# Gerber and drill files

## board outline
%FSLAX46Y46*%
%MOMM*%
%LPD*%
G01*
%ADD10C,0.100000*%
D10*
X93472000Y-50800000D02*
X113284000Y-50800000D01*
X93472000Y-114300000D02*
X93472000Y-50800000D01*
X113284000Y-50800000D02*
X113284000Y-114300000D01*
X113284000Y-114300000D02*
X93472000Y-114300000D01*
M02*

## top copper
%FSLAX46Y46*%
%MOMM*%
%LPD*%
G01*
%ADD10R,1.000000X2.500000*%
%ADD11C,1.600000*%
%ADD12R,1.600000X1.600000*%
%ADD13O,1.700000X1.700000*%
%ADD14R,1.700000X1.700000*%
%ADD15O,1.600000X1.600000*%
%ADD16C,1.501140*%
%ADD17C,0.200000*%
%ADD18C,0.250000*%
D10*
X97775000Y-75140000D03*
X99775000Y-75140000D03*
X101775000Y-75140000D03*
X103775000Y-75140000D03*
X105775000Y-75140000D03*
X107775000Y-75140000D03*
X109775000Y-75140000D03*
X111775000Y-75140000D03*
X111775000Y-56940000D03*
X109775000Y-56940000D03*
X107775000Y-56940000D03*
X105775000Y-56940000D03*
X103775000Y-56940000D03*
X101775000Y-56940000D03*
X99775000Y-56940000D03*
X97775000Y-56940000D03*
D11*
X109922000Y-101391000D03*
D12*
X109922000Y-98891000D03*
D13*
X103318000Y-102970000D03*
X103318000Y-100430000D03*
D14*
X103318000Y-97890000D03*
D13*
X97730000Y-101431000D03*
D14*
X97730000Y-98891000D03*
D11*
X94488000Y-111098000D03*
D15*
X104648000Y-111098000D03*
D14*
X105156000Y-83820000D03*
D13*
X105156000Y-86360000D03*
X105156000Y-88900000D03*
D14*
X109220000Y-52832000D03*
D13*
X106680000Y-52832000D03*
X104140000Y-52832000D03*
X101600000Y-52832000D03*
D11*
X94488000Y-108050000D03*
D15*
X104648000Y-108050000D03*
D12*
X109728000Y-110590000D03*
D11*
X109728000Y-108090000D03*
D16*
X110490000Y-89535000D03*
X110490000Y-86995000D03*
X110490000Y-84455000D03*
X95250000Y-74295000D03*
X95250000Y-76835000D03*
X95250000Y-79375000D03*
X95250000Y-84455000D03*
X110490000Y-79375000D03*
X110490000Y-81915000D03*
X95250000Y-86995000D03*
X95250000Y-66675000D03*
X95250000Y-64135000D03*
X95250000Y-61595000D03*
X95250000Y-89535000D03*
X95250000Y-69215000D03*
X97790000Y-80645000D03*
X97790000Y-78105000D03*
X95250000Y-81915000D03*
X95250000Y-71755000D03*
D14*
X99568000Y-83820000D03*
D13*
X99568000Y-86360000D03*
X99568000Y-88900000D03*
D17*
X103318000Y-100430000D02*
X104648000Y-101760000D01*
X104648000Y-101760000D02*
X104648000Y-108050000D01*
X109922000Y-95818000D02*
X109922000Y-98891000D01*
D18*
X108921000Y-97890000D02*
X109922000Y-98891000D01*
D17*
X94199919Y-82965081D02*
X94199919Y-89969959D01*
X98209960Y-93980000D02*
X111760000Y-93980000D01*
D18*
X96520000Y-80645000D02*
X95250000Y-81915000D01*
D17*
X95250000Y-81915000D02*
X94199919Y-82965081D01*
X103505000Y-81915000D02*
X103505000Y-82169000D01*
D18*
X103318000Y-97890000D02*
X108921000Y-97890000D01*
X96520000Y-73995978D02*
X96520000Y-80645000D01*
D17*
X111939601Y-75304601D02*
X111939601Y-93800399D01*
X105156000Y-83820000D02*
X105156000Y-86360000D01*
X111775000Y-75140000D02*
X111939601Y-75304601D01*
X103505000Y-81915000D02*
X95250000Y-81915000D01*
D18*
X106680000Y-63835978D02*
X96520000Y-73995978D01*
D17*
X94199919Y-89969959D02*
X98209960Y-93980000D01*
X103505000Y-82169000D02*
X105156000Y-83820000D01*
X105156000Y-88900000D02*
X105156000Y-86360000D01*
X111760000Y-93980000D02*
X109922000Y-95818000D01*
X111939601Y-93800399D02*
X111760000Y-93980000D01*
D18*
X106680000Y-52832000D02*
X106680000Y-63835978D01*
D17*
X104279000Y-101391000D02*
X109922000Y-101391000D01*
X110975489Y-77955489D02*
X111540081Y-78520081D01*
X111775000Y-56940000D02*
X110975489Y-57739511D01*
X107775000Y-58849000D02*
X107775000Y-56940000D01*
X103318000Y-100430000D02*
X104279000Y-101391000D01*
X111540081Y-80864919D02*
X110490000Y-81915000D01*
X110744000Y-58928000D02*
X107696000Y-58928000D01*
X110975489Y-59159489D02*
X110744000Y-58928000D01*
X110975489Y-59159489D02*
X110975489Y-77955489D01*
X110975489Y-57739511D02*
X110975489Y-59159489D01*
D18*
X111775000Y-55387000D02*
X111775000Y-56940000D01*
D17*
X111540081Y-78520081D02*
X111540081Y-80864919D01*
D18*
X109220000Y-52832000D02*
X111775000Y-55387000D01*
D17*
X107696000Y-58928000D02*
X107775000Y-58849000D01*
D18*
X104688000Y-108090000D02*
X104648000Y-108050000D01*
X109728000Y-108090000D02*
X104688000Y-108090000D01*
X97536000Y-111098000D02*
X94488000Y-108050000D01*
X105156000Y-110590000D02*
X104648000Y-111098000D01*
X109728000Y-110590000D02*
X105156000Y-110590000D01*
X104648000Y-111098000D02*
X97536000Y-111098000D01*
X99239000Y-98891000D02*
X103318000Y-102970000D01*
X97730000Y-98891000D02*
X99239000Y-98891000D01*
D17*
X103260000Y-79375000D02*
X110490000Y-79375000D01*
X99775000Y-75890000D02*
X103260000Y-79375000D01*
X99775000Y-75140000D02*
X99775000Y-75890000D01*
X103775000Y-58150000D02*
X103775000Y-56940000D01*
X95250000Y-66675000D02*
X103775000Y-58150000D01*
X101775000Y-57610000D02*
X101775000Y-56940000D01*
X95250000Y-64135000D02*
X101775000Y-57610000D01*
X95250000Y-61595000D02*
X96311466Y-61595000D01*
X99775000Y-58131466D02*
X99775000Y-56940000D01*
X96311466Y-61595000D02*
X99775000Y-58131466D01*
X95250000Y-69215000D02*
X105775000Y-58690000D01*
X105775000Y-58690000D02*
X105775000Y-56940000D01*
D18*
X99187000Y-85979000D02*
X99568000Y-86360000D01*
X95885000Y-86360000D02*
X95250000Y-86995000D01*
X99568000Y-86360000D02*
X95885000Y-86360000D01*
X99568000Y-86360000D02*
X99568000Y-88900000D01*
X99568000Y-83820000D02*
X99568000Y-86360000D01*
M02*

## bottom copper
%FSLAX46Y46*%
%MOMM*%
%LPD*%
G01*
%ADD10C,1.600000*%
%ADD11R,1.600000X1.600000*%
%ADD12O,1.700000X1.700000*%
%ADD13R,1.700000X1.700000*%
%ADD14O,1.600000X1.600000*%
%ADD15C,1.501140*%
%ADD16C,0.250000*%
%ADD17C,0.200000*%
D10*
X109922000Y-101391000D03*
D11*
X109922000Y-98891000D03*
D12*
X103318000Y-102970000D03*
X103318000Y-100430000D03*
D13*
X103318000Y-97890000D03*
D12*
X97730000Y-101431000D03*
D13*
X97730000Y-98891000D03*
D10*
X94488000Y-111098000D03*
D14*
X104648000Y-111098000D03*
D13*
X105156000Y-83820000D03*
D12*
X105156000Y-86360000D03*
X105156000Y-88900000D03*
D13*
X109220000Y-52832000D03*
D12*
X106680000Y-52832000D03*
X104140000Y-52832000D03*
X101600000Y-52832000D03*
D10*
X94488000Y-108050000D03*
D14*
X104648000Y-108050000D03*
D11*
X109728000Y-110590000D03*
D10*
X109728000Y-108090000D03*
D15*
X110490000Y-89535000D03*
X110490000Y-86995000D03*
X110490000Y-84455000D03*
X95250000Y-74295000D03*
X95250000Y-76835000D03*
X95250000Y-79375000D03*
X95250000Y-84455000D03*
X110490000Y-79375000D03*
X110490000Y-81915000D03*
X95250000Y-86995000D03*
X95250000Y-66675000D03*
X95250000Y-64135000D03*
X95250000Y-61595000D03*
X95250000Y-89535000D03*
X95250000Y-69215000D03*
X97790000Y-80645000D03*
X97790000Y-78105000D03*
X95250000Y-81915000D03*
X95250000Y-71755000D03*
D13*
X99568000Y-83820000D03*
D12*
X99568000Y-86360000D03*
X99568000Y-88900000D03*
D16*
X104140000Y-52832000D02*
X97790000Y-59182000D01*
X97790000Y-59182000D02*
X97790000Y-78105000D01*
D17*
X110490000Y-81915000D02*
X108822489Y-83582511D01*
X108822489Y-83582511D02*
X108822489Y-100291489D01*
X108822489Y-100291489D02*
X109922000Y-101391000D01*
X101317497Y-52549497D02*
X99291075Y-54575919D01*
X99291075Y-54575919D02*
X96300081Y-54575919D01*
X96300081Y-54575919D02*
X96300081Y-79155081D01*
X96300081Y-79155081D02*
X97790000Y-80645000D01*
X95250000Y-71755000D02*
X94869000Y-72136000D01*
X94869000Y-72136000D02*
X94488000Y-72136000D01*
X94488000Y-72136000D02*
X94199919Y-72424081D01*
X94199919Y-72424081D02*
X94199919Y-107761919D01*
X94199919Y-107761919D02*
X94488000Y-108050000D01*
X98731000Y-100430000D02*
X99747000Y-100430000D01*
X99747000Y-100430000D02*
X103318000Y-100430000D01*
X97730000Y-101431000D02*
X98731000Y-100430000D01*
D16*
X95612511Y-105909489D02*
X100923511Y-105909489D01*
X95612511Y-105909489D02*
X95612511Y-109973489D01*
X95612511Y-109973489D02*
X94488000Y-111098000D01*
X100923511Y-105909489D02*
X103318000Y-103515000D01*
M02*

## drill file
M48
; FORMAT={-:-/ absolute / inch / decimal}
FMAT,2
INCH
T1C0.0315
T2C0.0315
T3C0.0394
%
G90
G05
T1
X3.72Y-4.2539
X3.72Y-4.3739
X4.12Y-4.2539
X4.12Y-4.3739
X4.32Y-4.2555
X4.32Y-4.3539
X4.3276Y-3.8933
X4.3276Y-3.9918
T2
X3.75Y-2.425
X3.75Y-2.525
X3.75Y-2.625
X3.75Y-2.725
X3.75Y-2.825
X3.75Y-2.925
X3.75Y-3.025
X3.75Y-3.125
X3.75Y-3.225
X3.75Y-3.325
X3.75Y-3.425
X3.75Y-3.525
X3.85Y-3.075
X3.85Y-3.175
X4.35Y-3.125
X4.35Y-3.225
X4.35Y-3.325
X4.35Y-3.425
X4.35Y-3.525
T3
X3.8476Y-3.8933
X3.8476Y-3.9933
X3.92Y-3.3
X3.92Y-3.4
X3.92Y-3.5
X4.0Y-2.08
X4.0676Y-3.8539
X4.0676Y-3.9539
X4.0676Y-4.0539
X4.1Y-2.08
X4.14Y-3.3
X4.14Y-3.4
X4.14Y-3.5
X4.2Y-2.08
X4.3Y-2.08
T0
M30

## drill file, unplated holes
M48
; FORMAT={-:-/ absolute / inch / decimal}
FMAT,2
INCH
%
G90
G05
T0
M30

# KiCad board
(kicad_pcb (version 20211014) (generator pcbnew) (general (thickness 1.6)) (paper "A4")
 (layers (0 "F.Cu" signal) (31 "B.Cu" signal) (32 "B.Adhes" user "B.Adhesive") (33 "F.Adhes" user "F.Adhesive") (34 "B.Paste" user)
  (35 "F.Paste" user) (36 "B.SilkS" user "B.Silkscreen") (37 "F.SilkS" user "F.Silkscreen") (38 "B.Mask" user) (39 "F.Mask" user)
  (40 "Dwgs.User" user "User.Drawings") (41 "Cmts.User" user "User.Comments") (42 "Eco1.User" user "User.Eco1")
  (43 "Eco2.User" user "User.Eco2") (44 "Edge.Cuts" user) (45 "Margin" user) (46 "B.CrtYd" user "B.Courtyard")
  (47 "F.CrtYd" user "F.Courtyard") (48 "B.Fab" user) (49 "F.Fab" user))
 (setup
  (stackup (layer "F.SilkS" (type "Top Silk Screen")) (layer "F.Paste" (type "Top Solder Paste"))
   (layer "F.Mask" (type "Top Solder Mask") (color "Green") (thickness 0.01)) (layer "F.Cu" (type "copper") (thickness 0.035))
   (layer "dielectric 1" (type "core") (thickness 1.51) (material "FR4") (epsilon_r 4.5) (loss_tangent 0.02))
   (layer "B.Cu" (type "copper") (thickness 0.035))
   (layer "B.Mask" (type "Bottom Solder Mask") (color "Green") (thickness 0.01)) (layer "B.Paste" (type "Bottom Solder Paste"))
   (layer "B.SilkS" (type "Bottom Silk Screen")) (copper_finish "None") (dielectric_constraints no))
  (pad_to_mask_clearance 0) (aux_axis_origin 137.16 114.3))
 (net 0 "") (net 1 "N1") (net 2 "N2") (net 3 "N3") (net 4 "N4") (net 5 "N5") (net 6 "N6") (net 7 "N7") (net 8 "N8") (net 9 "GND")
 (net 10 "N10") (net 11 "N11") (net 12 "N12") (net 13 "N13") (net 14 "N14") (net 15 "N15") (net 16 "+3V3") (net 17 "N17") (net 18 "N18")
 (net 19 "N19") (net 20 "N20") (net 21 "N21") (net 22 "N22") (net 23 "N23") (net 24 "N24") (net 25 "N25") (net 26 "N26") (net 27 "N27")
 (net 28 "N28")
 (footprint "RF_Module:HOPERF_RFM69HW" (layer "F.Cu") (at 104.775 66.04 90)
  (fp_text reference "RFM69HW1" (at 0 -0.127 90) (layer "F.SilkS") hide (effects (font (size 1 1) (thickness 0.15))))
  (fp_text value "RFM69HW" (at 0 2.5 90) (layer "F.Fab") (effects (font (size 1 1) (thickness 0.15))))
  (pad "1" smd rect (at -9.1 -7 90) (size 2.5 1) (layers "F.Cu" "F.Paste" "F.Mask") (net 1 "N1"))
  (pad "2" smd rect (at -9.1 -5 90) (size 2.5 1) (layers "F.Cu" "F.Paste" "F.Mask") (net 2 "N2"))
  (pad "3" smd rect (at -9.1 -3 90) (size 2.5 1) (layers "F.Cu" "F.Paste" "F.Mask") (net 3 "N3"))
  (pad "4" smd rect (at -9.1 -1 90) (size 2.5 1) (layers "F.Cu" "F.Paste" "F.Mask") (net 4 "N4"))
  (pad "5" smd rect (at -9.1 1 90) (size 2.5 1) (layers "F.Cu" "F.Paste" "F.Mask") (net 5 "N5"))
  (pad "6" smd rect (at -9.1 3 90) (size 2.5 1) (layers "F.Cu" "F.Paste" "F.Mask") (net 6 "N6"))
  (pad "7" smd rect (at -9.1 5 90) (size 2.5 1) (layers "F.Cu" "F.Paste" "F.Mask") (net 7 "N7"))
  (pad "8" smd rect (at -9.1 7 90) (size 2.5 1) (layers "F.Cu" "F.Paste" "F.Mask") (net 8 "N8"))
  (pad "9" smd rect (at 9.1 7 90) (size 2.5 1) (layers "F.Cu" "F.Paste" "F.Mask") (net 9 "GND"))
  (pad "10" smd rect (at 9.1 5 90) (size 2.5 1) (layers "F.Cu" "F.Paste" "F.Mask") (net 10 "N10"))
  (pad "11" smd rect (at 9.1 3 90) (size 2.5 1) (layers "F.Cu" "F.Paste" "F.Mask") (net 9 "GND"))
  (pad "12" smd rect (at 9.1 1 90) (size 2.5 1) (layers "F.Cu" "F.Paste" "F.Mask") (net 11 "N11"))
  (pad "13" smd rect (at 9.1 -1 90) (size 2.5 1) (layers "F.Cu" "F.Paste" "F.Mask") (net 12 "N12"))
  (pad "14" smd rect (at 9.1 -3 90) (size 2.5 1) (layers "F.Cu" "F.Paste" "F.Mask") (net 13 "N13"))
  (pad "15" smd rect (at 9.1 -5 90) (size 2.5 1) (layers "F.Cu" "F.Paste" "F.Mask") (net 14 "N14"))
  (pad "16" smd rect (at 9.1 -7 90) (size 2.5 1) (layers "F.Cu" "F.Paste" "F.Mask") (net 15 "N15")))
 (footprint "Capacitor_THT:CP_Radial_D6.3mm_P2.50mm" (layer "F.Cu") (at 109.922 98.891 -90)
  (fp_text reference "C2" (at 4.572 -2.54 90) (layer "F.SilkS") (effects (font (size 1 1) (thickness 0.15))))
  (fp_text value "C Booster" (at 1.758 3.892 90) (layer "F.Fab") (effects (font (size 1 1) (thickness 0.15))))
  (pad "1" thru_hole rect (at 0 0 270) (size 1.6 1.6) (drill 0.8) (layers *.Cu *.Mask) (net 8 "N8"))
  (pad "2" thru_hole circle (at 2.5 0 270) (size 1.6 1.6) (drill 0.8) (layers *.Cu *.Mask) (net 9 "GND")))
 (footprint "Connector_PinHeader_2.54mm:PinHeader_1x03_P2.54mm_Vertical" (layer "F.Cu") (at 103.318 97.89)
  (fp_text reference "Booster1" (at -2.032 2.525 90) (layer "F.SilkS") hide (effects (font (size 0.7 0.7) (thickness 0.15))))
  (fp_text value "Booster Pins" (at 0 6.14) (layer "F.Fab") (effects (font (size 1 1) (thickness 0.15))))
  (pad "1" thru_hole rect (at 0 0) (size 1.7 1.7) (drill 1) (layers *.Cu *.Mask) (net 8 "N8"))
  (pad "2" thru_hole oval (at 0 2.54) (size 1.7 1.7) (drill 1) (layers *.Cu *.Mask) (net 9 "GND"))
  (pad "3" thru_hole oval (at 0 5.08) (size 1.7 1.7) (drill 1) (layers *.Cu *.Mask) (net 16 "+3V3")))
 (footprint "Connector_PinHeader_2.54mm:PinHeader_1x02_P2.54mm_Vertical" (layer "F.Cu") (at 97.73 98.891)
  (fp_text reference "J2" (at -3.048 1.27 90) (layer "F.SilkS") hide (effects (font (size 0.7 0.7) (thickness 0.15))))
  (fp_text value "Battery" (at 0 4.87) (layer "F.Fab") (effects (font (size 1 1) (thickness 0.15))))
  (pad "1" thru_hole rect (at 0 0) (size 1.7 1.7) (drill 1) (layers *.Cu *.Mask) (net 16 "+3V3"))
  (pad "2" thru_hole oval (at 0 2.54) (size 1.7 1.7) (drill 1) (layers *.Cu *.Mask) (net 9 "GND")))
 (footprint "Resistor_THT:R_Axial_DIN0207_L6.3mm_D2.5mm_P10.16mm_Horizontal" (layer "F.Cu") (at 94.488 111.098)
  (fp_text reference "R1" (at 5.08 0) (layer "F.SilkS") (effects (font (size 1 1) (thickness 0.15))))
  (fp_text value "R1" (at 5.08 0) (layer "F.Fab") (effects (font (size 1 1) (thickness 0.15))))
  (pad "1" thru_hole circle (at 0 0) (size 1.6 1.6) (drill 0.8) (layers *.Cu *.Mask) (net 16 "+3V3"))
  (pad "2" thru_hole oval (at 10.16 0) (size 1.6 1.6) (drill 0.8) (layers *.Cu *.Mask) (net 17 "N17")))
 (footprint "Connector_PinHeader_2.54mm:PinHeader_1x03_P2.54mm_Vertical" (layer "F.Cu") (at 105.156 83.82)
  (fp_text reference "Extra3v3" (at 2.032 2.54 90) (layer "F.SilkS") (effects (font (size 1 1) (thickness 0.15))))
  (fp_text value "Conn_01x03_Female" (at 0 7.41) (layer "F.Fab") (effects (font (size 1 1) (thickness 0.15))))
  (pad "1" thru_hole rect (at 0 0) (size 1.7 1.7) (drill 1) (layers *.Cu *.Mask) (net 8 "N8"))
  (pad "2" thru_hole oval (at 0 2.54) (size 1.7 1.7) (drill 1) (layers *.Cu *.Mask) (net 8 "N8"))
  (pad "3" thru_hole oval (at 0 5.08) (size 1.7 1.7) (drill 1) (layers *.Cu *.Mask) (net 8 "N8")))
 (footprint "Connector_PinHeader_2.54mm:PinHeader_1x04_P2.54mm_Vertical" (layer "F.Cu") (at 109.22 52.832 -90)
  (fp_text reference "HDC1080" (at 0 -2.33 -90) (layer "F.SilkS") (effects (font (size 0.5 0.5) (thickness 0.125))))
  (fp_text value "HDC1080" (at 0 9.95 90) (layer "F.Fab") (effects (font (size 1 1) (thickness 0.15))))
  (pad "1" thru_hole rect (at 0 0 270) (size 1.7 1.7) (drill 1) (layers *.Cu *.Mask) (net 9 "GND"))
  (pad "2" thru_hole oval (at 0 2.54 270) (size 1.7 1.7) (drill 1) (layers *.Cu *.Mask) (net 8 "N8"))
  (pad "3" thru_hole oval (at 0 5.08 270) (size 1.7 1.7) (drill 1) (layers *.Cu *.Mask) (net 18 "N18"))
  (pad "4" thru_hole oval (at 0 7.62 270) (size 1.7 1.7) (drill 1) (layers *.Cu *.Mask) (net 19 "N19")))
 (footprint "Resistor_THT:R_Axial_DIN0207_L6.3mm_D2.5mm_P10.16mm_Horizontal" (layer "F.Cu") (at 94.488 108.05)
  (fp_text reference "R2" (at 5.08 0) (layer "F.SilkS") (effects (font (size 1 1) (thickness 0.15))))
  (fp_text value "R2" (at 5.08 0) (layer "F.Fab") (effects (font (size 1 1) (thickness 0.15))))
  (pad "1" thru_hole circle (at 0 0) (size 1.6 1.6) (drill 0.8) (layers *.Cu *.Mask) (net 17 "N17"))
  (pad "2" thru_hole oval (at 10.16 0) (size 1.6 1.6) (drill 0.8) (layers *.Cu *.Mask) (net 9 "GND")))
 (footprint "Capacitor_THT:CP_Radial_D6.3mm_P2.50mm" (layer "F.Cu") (at 109.728 110.59 90)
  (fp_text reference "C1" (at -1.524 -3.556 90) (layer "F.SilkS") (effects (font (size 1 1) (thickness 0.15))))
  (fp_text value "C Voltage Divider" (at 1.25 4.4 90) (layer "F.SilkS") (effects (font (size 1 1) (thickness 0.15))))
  (pad "1" thru_hole rect (at 0 0 90) (size 1.6 1.6) (drill 0.8) (layers *.Cu *.Mask) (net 17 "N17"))
  (pad "2" thru_hole circle (at 2.5 0 90) (size 1.6 1.6) (drill 0.8) (layers *.Cu *.Mask) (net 9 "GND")))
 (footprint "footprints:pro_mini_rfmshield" (layer "F.Cu") (at 102.87 75.565)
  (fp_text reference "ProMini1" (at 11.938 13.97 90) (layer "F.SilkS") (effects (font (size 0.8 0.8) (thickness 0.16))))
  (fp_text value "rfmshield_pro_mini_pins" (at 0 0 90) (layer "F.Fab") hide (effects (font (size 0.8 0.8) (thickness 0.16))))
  (pad "1" thru_hole circle (at 7.62 13.97 90) (size 1.50114 1.50114) (drill 0.8001) (layers *.Cu *.Mask "F.SilkS") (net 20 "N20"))
  (pad "2" thru_hole circle (at 7.62 11.43 90) (size 1.50114 1.50114) (drill 0.8001) (layers *.Cu *.Mask "F.SilkS") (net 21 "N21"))
  (pad "3" thru_hole circle (at 7.62 8.89 90) (size 1.50114 1.50114) (drill 0.8001) (layers *.Cu *.Mask "F.SilkS") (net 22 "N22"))
  (pad "18" thru_hole circle (at -7.62 -1.27 90) (size 1.50114 1.50114) (drill 0.8001) (layers *.Cu *.Mask "F.SilkS") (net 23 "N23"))
  (pad "19" thru_hole circle (at -7.62 1.27 90) (size 1.50114 1.50114) (drill 0.8001) (layers *.Cu *.Mask "F.SilkS") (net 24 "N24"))
  (pad "20" thru_hole circle (at -7.62 3.81 90) (size 1.50114 1.50114) (drill 0.8001) (layers *.Cu *.Mask "F.SilkS") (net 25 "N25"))
  (pad "22" thru_hole circle (at -7.62 8.89 90) (size 1.50114 1.50114) (drill 0.8001) (layers *.Cu *.Mask "F.SilkS") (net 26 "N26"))
  (pad "DI00" thru_hole circle (at 7.62 3.81 90) (size 1.50114 1.50114) (drill 0.8001) (layers *.Cu *.Mask "F.SilkS") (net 2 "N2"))
  (pad "GND1" thru_hole circle (at 7.62 6.35 90) (size 1.50114 1.50114) (drill 0.8001) (layers *.Cu *.Mask "F.SilkS") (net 9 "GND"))
  (pad "GND2" thru_hole circle (at -7.62 11.43 90) (size 1.50114 1.50114) (drill 0.8001) (layers *.Cu *.Mask "F.SilkS") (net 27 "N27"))
  (pad "MISO" thru_hole circle (at -7.62 -8.89 90) (size 1.50114 1.50114) (drill 0.8001) (layers *.Cu *.Mask "F.SilkS") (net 12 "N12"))
  (pad "MOSI" thru_hole circle (at -7.62 -11.43 90) (size 1.50114 1.50114) (drill 0.8001) (layers *.Cu *.Mask "F.SilkS") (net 13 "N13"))
  (pad "NSS" thru_hole circle (at -7.62 -13.97 90) (size 1.50114 1.50114) (drill 0.8001) (layers *.Cu *.Mask "F.SilkS") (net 14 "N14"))
  (pad "RAW" thru_hole circle (at -7.62 13.97 90) (size 1.50114 1.50114) (drill 0.8001) (layers *.Cu *.Mask "F.SilkS") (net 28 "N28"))
  (pad "SCK" thru_hole circle (at -7.62 -6.35 90) (size 1.50114 1.50114) (drill 0.8001) (layers *.Cu *.Mask "F.SilkS") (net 11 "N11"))
  (pad "SCL" thru_hole circle (at -5.08 5.08 90) (size 1.50114 1.50114) (drill 0.8001) (layers *.Cu *.Mask "F.SilkS") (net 19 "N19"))
  (pad "SDA" thru_hole circle (at -5.08 2.54 90) (size 1.50114 1.50114) (drill 0.8001) (layers *.Cu *.Mask "F.SilkS") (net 18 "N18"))
  (pad "VCC" thru_hole circle (at -7.62 6.35 90) (size 1.50114 1.50114) (drill 0.8001) (layers *.Cu *.Mask "F.SilkS") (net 8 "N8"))
  (pad "VolDiv" thru_hole circle (at -7.62 -3.81 90) (size 1.50114 1.50114) (drill 0.8001) (layers *.Cu *.Mask "F.SilkS") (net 17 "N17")))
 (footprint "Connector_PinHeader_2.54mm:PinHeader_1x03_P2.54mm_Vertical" (layer "F.Cu") (at 99.568 83.82)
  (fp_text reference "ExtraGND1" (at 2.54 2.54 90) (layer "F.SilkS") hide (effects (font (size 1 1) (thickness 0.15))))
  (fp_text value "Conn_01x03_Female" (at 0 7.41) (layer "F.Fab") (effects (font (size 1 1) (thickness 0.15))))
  (pad "1" thru_hole rect (at 0 0) (size 1.7 1.7) (drill 1) (layers *.Cu *.Mask) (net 27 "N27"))
  (pad "2" thru_hole oval (at 0 2.54) (size 1.7 1.7) (drill 1) (layers *.Cu *.Mask) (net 27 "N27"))
  (pad "3" thru_hole oval (at 0 5.08) (size 1.7 1.7) (drill 1) (layers *.Cu *.Mask) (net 27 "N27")))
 (gr_line (start 93.472 50.8) (end 113.284 50.8) (layer "Edge.Cuts") (width 0.1))
 (gr_line (start 93.472 114.3) (end 93.472 50.8) (layer "Edge.Cuts") (width 0.1))
 (gr_line (start 113.284 50.8) (end 113.284 114.3) (layer "Edge.Cuts") (width 0.1))
 (gr_line (start 113.284 114.3) (end 93.472 114.3) (layer "Edge.Cuts") (width 0.1))
 (segment (start 109.922 95.818) (end 109.922 98.891) (width 0.2) (layer "F.Cu") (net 8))
 (segment (start 108.921 97.89) (end 109.922 98.891) (width 0.25) (layer "F.Cu") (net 8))
 (segment (start 94.199919 82.965081) (end 94.199919 89.969959) (width 0.2) (layer "F.Cu") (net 8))
 (segment (start 98.20996 93.98) (end 111.76 93.98) (width 0.2) (layer "F.Cu") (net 8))
 (segment (start 96.52 80.645) (end 95.25 81.915) (width 0.25) (layer "F.Cu") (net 8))
 (segment (start 95.25 81.915) (end 94.199919 82.965081) (width 0.2) (layer "F.Cu") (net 8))
 (segment (start 103.505 81.915) (end 103.505 82.169) (width 0.2) (layer "F.Cu") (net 8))
 (segment (start 103.318 97.89) (end 108.921 97.89) (width 0.25) (layer "F.Cu") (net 8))
 (segment (start 96.52 73.995978) (end 96.52 80.645) (width 0.25) (layer "F.Cu") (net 8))
 (segment (start 111.939601 75.304601) (end 111.939601 93.800399) (width 0.2) (layer "F.Cu") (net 8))
 (segment (start 105.156 83.82) (end 105.156 86.36) (width 0.2) (layer "F.Cu") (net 8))
 (segment (start 111.775 75.14) (end 111.939601 75.304601) (width 0.2) (layer "F.Cu") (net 8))
 (segment (start 103.505 81.915) (end 95.25 81.915) (width 0.2) (layer "F.Cu") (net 8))
 (segment (start 106.68 63.835978) (end 96.52 73.995978) (width 0.25) (layer "F.Cu") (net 8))
 (segment (start 94.199919 89.969959) (end 98.20996 93.98) (width 0.2) (layer "F.Cu") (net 8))
 (segment (start 103.505 82.169) (end 105.156 83.82) (width 0.2) (layer "F.Cu") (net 8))
 (segment (start 105.156 88.9) (end 105.156 86.36) (width 0.2) (layer "F.Cu") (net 8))
 (segment (start 111.76 93.98) (end 109.922 95.818) (width 0.2) (layer "F.Cu") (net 8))
 (segment (start 111.939601 93.800399) (end 111.76 93.98) (width 0.2) (layer "F.Cu") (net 8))
 (segment (start 106.68 52.832) (end 106.68 63.835978) (width 0.25) (layer "F.Cu") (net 8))
 (segment (start 104.279 101.391) (end 109.922 101.391) (width 0.2) (layer "F.Cu") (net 9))
 (segment (start 110.975489 77.955489) (end 111.540081 78.520081) (width 0.2) (layer "F.Cu") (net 9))
 (segment (start 111.775 56.94) (end 110.975489 57.739511) (width 0.2) (layer "F.Cu") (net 9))
 (segment (start 107.775 58.849) (end 107.775 56.94) (width 0.2) (layer "F.Cu") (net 9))
 (segment (start 103.318 100.43) (end 104.648 101.76) (width 0.2) (layer "F.Cu") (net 9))
 (segment (start 103.318 100.43) (end 104.279 101.391) (width 0.2) (layer "F.Cu") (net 9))
 (segment (start 111.540081 80.864919) (end 110.49 81.915) (width 0.2) (layer "F.Cu") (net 9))
 (segment (start 110.744 58.928) (end 107.696 58.928) (width 0.2) (layer "F.Cu") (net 9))
 (segment (start 110.975489 59.159489) (end 110.744 58.928) (width 0.2) (layer "F.Cu") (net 9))
 (segment (start 110.975489 59.159489) (end 110.975489 77.955489) (width 0.2) (layer "F.Cu") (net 9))
 (segment (start 110.975489 57.739511) (end 110.975489 59.159489) (width 0.2) (layer "F.Cu") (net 9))
 (segment (start 111.775 55.387) (end 111.775 56.94) (width 0.25) (layer "F.Cu") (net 9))
 (segment (start 111.540081 78.520081) (end 111.540081 80.864919) (width 0.2) (layer "F.Cu") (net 9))
 (segment (start 104.648 101.76) (end 104.648 108.05) (width 0.2) (layer "F.Cu") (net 9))
 (segment (start 109.22 52.832) (end 111.775 55.387) (width 0.25) (layer "F.Cu") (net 9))
 (segment (start 107.696 58.928) (end 107.775 58.849) (width 0.2) (layer "F.Cu") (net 9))
 (segment (start 104.688 108.09) (end 104.648 108.05) (width 0.25) (layer "F.Cu") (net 9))
 (segment (start 109.728 108.09) (end 104.688 108.09) (width 0.25) (layer "F.Cu") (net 9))
 (segment (start 98.731 100.43) (end 99.747 100.43) (width 0.2) (layer "B.Cu") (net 9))
 (segment (start 99.747 100.43) (end 103.318 100.43) (width 0.2) (layer "B.Cu") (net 9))
 (segment (start 110.49 81.915) (end 108.822489 83.582511) (width 0.2) (layer "B.Cu") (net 9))
 (segment (start 108.822489 100.291489) (end 109.922 101.391) (width 0.2) (layer "B.Cu") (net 9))
 (segment (start 108.822489 83.582511) (end 108.822489 100.291489) (width 0.2) (layer "B.Cu") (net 9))
 (segment (start 97.73 101.431) (end 98.731 100.43) (width 0.2) (layer "B.Cu") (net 9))
 (segment (start 97.536 111.098) (end 94.488 108.05) (width 0.25) (layer "F.Cu") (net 17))
 (segment (start 105.156 110.59) (end 104.648 111.098) (width 0.25) (layer "F.Cu") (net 17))
 (segment (start 109.728 110.59) (end 105.156 110.59) (width 0.25) (layer "F.Cu") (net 17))
 (segment (start 104.648 111.098) (end 97.536 111.098) (width 0.25) (layer "F.Cu") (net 17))
 (segment (start 94.869 72.136) (end 94.488 72.136) (width 0.2) (layer "B.Cu") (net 17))
 (segment (start 94.199919 107.761919) (end 94.488 108.05) (width 0.2) (layer "B.Cu") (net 17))
 (segment (start 94.488 72.136) (end 94.199919 72.424081) (width 0.2) (layer "B.Cu") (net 17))
 (segment (start 94.199919 72.424081) (end 94.199919 107.761919) (width 0.2) (layer "B.Cu") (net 17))
 (segment (start 95.25 71.755) (end 94.869 72.136) (width 0.2) (layer "B.Cu") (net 17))
 (segment (start 99.239 98.891) (end 103.318 102.97) (width 0.25) (layer "F.Cu") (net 16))
 (segment (start 97.73 98.891) (end 99.239 98.891) (width 0.25) (layer "F.Cu") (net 16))
 (segment (start 95.612511 105.909489) (end 100.923511 105.909489) (width 0.25) (layer "B.Cu") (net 16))
 (segment (start 95.612511 105.909489) (end 95.612511 109.973489) (width 0.25) (layer "B.Cu") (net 16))
 (segment (start 95.612511 109.973489) (end 94.488 111.098) (width 0.25) (layer "B.Cu") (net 16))
 (segment (start 100.923511 105.909489) (end 103.318 103.515) (width 0.25) (layer "B.Cu") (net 16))
 (segment (start 103.26 79.375) (end 110.49 79.375) (width 0.2) (layer "F.Cu") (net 2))
 (segment (start 99.775 75.89) (end 103.26 79.375) (width 0.2) (layer "F.Cu") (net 2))
 (segment (start 99.775 75.14) (end 99.775 75.89) (width 0.2) (layer "F.Cu") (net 2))
 (segment (start 103.775 58.15) (end 103.775 56.94) (width 0.2) (layer "F.Cu") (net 12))
 (segment (start 95.25 66.675) (end 103.775 58.15) (width 0.2) (layer "F.Cu") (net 12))
 (segment (start 101.775 57.61) (end 101.775 56.94) (width 0.2) (layer "F.Cu") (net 13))
 (segment (start 95.25 64.135) (end 101.775 57.61) (width 0.2) (layer "F.Cu") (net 13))
 (segment (start 95.25 61.595) (end 96.311466 61.595) (width 0.2) (layer "F.Cu") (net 14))
 (segment (start 99.775 58.131466) (end 99.775 56.94) (width 0.2) (layer "F.Cu") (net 14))
 (segment (start 96.311466 61.595) (end 99.775 58.131466) (width 0.2) (layer "F.Cu") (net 14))
 (segment (start 95.25 69.215) (end 105.775 58.69) (width 0.2) (layer "F.Cu") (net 11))
 (segment (start 105.775 58.69) (end 105.775 56.94) (width 0.2) (layer "F.Cu") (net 11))
 (segment (start 104.14 52.832) (end 97.79 59.182) (width 0.25) (layer "B.Cu") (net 18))
 (segment (start 97.79 59.182) (end 97.79 78.105) (width 0.25) (layer "B.Cu") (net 18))
 (segment (start 96.300081 79.155081) (end 97.79 80.645) (width 0.2) (layer "B.Cu") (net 19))
 (segment (start 101.317497 52.549497) (end 99.291075 54.575919) (width 0.2) (layer "B.Cu") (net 19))
 (segment (start 96.300081 54.575919) (end 96.300081 79.155081) (width 0.2) (layer "B.Cu") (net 19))
 (segment (start 99.291075 54.575919) (end 96.300081 54.575919) (width 0.2) (layer "B.Cu") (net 19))
 (segment (start 99.187 85.979) (end 99.568 86.36) (width 0.25) (layer "F.Cu") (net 27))
 (segment (start 95.885 86.36) (end 95.25 86.995) (width 0.25) (layer "F.Cu") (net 27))
 (segment (start 99.568 86.36) (end 95.885 86.36) (width 0.25) (layer "F.Cu") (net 27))
 (segment (start 99.568 86.36) (end 99.568 88.9) (width 0.25) (layer "F.Cu") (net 27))
 (segment (start 99.568 83.82) (end 99.568 86.36) (width 0.25) (layer "F.Cu") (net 27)))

